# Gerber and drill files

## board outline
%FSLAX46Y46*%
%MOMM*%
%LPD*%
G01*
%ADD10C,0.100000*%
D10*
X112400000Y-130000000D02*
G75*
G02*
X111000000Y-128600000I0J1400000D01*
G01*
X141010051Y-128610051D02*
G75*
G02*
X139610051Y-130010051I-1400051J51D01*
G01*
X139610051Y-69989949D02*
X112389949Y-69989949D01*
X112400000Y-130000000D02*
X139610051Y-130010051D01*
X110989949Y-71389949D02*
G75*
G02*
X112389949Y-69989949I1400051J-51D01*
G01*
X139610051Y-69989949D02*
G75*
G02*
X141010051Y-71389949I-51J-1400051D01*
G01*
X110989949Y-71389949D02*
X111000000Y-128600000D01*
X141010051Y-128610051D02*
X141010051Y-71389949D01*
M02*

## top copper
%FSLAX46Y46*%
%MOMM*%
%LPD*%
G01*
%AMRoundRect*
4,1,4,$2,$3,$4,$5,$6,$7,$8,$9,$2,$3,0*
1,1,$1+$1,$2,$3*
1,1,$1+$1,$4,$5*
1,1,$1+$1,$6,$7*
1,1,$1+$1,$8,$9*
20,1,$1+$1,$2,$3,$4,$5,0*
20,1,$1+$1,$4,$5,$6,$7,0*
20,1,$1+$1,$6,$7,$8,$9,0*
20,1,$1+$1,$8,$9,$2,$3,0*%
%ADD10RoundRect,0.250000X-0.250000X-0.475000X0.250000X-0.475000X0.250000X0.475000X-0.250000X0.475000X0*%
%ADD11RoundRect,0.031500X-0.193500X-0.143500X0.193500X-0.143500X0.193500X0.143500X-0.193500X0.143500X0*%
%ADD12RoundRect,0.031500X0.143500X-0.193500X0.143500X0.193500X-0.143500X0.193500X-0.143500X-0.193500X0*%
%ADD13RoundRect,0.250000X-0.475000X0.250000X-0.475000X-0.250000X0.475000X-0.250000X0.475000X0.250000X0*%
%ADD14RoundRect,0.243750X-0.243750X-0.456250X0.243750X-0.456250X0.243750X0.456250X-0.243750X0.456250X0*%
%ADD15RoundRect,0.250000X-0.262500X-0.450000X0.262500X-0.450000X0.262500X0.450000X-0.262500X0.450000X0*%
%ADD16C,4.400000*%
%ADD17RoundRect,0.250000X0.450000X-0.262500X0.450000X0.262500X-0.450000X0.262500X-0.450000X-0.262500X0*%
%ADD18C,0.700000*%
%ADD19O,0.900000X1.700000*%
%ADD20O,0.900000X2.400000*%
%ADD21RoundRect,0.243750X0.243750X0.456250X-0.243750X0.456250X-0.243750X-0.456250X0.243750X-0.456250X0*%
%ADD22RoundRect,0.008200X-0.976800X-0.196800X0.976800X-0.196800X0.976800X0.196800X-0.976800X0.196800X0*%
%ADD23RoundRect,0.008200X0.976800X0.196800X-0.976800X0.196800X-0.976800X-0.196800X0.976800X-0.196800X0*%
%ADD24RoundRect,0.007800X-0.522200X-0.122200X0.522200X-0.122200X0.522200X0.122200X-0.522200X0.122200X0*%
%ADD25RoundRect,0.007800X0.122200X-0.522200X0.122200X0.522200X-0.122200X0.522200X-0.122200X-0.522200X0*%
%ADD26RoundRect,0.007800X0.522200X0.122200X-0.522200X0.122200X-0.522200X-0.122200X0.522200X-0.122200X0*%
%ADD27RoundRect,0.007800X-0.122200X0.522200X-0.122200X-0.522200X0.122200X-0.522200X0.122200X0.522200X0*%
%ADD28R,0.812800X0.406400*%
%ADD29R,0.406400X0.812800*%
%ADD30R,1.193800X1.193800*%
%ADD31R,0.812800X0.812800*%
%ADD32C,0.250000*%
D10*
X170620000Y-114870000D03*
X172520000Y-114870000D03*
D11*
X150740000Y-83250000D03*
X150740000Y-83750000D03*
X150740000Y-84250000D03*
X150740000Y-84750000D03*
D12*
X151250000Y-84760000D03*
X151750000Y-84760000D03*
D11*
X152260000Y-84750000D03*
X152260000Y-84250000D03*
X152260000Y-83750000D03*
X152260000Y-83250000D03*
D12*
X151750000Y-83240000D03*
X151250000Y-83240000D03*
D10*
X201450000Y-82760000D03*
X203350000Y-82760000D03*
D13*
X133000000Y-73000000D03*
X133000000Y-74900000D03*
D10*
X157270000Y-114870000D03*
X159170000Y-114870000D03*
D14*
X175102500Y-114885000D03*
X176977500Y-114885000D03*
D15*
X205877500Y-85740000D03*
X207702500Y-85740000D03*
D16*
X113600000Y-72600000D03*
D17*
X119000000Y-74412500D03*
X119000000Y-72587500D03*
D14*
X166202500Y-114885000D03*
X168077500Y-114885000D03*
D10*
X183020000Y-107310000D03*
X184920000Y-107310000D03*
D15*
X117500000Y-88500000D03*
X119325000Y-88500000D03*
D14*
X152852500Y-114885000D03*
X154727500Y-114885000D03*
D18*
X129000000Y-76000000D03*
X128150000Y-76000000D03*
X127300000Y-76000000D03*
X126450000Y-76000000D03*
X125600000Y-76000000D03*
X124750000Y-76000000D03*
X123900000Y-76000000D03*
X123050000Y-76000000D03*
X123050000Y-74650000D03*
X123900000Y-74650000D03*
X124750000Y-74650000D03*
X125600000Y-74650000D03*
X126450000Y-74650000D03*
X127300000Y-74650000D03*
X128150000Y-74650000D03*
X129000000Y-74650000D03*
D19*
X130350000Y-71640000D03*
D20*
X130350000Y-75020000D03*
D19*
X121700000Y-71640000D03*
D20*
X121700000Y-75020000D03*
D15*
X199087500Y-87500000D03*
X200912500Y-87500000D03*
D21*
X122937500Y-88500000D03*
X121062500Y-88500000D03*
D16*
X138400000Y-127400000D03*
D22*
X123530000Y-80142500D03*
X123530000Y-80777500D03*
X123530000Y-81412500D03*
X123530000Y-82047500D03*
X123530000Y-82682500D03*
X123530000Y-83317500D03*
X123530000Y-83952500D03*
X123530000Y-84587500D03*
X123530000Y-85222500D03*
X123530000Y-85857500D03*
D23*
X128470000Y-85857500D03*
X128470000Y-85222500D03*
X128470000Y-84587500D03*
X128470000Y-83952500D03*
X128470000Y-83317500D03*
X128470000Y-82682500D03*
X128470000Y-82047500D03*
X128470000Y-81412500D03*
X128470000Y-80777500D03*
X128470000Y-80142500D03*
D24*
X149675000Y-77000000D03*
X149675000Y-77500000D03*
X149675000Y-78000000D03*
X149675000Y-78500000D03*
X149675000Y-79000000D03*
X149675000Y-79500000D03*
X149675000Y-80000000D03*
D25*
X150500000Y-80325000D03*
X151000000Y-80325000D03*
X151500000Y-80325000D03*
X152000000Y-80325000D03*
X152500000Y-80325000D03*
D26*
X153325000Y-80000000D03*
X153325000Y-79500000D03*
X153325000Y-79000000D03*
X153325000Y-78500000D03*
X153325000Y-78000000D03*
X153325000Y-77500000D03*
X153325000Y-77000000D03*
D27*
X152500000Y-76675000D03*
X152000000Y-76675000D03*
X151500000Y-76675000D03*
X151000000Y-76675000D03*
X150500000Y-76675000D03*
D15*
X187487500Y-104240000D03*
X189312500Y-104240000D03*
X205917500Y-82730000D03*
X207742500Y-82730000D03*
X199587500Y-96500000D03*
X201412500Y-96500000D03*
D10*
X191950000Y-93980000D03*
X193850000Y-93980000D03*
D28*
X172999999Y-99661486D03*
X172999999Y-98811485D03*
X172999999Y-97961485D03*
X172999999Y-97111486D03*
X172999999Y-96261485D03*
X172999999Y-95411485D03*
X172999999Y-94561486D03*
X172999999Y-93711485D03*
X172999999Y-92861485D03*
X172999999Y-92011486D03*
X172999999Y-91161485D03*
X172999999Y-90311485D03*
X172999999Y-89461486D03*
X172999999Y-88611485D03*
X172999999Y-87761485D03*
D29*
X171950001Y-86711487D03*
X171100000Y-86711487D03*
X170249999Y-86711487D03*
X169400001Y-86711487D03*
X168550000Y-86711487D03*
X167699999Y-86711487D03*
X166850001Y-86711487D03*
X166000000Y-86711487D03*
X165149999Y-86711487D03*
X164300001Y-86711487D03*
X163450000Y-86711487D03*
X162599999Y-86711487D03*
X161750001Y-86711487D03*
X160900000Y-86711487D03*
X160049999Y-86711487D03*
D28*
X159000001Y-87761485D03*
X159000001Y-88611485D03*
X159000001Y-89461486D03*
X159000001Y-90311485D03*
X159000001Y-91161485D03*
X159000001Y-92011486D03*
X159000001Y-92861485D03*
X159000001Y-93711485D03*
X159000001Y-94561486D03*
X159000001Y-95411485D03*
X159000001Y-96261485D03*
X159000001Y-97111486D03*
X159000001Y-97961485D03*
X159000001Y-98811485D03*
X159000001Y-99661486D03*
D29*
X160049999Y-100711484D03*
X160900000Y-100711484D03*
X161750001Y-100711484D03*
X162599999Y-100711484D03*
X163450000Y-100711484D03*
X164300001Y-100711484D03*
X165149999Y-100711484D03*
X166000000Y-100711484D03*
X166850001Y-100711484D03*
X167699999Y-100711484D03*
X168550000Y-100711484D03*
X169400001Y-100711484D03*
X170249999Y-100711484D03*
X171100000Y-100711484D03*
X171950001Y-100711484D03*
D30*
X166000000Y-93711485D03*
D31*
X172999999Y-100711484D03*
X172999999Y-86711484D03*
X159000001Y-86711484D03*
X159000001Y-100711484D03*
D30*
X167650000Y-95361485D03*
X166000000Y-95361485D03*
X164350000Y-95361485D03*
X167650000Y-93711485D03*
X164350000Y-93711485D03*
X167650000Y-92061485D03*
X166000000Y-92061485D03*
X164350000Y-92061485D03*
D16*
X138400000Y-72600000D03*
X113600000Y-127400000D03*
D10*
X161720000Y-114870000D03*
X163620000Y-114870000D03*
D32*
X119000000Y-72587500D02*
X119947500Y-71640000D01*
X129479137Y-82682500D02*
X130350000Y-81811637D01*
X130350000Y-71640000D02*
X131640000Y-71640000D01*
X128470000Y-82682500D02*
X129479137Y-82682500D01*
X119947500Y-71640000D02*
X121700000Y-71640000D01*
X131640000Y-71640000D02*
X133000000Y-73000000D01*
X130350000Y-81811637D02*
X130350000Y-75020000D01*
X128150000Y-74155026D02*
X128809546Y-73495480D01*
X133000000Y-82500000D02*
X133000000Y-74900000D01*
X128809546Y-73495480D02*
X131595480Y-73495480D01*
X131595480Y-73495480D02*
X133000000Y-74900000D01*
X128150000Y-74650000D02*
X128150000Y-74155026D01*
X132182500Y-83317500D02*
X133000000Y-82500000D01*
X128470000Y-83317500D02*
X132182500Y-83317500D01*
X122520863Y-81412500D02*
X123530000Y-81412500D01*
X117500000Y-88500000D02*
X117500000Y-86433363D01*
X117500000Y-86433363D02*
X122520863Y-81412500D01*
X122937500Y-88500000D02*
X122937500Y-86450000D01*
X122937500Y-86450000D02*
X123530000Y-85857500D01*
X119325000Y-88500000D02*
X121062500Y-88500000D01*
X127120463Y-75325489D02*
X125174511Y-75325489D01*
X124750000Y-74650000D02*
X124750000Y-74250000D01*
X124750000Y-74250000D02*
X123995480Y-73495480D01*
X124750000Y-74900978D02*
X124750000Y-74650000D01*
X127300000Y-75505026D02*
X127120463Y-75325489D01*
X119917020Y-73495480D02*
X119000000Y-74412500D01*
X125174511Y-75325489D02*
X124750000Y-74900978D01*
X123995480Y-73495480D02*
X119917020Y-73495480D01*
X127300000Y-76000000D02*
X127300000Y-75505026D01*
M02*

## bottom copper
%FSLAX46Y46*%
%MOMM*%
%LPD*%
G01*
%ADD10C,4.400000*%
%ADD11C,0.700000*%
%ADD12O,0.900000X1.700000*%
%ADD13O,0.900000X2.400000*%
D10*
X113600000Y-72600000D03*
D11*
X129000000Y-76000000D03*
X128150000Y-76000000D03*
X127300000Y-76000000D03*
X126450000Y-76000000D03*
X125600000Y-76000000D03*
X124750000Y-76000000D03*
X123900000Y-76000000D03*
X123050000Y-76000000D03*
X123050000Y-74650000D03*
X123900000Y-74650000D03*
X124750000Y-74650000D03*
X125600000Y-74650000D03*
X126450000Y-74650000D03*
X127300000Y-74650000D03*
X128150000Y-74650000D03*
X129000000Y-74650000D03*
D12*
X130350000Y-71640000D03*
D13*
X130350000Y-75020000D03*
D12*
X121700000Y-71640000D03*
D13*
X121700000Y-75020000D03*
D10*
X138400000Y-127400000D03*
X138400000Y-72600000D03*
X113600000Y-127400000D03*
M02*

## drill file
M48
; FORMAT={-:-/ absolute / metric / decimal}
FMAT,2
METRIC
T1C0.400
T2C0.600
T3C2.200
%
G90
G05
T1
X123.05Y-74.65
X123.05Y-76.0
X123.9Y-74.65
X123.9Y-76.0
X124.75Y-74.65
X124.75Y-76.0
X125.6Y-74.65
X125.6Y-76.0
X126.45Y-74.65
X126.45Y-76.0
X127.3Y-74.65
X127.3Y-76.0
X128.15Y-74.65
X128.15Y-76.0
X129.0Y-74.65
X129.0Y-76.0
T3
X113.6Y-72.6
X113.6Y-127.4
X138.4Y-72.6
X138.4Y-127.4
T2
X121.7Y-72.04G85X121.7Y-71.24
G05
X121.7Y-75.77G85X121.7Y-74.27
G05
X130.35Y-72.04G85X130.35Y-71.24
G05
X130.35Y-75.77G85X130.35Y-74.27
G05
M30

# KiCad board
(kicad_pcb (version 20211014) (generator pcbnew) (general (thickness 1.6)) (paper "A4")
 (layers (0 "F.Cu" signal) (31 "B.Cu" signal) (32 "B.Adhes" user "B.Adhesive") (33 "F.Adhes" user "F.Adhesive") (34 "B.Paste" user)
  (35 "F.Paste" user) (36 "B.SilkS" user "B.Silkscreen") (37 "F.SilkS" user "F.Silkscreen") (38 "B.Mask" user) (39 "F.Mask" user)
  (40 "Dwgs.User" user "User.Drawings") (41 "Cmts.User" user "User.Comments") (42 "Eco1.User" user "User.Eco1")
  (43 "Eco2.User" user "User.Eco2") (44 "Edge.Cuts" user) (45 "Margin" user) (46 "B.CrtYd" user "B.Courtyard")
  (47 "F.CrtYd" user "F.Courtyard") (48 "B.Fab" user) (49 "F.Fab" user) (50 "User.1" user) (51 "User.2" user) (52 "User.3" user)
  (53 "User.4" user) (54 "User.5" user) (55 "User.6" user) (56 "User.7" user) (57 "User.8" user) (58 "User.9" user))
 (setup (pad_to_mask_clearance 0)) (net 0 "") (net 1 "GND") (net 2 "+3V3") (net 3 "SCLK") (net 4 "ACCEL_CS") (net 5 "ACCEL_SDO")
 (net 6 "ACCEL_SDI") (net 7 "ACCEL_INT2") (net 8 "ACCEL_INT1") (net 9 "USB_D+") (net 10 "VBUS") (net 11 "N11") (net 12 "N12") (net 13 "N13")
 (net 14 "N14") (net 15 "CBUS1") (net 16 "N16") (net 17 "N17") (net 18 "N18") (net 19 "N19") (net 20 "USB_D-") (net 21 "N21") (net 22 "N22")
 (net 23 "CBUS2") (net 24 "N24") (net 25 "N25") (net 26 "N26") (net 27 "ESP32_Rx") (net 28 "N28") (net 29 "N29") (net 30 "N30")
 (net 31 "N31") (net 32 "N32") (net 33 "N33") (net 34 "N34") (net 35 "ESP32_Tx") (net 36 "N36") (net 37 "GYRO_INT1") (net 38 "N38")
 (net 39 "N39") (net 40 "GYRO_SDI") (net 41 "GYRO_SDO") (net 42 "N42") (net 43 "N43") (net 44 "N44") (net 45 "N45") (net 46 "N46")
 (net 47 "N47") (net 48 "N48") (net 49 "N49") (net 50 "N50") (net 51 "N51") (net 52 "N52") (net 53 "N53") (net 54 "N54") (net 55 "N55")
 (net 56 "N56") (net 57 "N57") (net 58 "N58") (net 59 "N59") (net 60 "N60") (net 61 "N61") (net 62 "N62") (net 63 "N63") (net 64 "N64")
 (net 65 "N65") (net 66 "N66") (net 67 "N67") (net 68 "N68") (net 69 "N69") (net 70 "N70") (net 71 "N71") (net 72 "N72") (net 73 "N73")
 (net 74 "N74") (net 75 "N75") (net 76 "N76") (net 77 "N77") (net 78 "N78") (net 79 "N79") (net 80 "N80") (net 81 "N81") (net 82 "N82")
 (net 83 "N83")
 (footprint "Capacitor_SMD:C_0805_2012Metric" (layer "F.Cu") (at 171.57 114.87)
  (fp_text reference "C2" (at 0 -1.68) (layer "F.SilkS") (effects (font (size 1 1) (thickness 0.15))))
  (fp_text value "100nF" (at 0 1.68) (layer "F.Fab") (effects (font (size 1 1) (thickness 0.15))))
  (pad "1" smd roundrect (at -0.95 0) (size 1 1.45) (layers "F.Cu" "F.Paste" "F.Mask") (roundrect_rratio 0.25) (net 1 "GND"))
  (pad "2" smd roundrect (at 0.95 0) (size 1 1.45) (layers "F.Cu" "F.Paste" "F.Mask") (roundrect_rratio 0.25) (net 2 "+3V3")))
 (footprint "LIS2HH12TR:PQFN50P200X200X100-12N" (layer "F.Cu") (at 151.5 84)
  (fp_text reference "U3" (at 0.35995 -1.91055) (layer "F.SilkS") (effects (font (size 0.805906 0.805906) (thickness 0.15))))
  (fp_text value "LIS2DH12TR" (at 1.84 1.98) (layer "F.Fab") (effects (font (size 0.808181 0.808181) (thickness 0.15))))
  (pad "1" smd roundrect locked (at -0.76 -0.75) (size 0.45 0.35) (layers "F.Cu" "F.Paste" "F.Mask") (roundrect_rratio 0.09) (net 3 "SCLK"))
  (pad "2" smd roundrect locked (at -0.76 -0.25) (size 0.45 0.35) (layers "F.Cu" "F.Paste" "F.Mask") (roundrect_rratio 0.09)
   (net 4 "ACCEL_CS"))
  (pad "3" smd roundrect locked (at -0.76 0.25) (size 0.45 0.35) (layers "F.Cu" "F.Paste" "F.Mask") (roundrect_rratio 0.09)
   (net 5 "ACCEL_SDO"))
  (pad "4" smd roundrect locked (at -0.76 0.75) (size 0.45 0.35) (layers "F.Cu" "F.Paste" "F.Mask") (roundrect_rratio 0.09)
   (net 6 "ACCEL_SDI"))
  (pad "5" smd roundrect locked (at -0.25 0.76 90) (size 0.45 0.35) (layers "F.Cu" "F.Paste" "F.Mask") (roundrect_rratio 0.09) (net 1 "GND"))
  (pad "6" smd roundrect locked (at 0.25 0.76 90) (size 0.45 0.35) (layers "F.Cu" "F.Paste" "F.Mask") (roundrect_rratio 0.09) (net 1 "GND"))
  (pad "7" smd roundrect locked (at 0.76 0.75) (size 0.45 0.35) (layers "F.Cu" "F.Paste" "F.Mask") (roundrect_rratio 0.09) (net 1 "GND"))
  (pad "8" smd roundrect locked (at 0.76 0.25) (size 0.45 0.35) (layers "F.Cu" "F.Paste" "F.Mask") (roundrect_rratio 0.09) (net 1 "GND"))
  (pad "9" smd roundrect locked (at 0.76 -0.25) (size 0.45 0.35) (layers "F.Cu" "F.Paste" "F.Mask") (roundrect_rratio 0.09) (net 2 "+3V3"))
  (pad "10" smd roundrect locked (at 0.76 -0.75) (size 0.45 0.35) (layers "F.Cu" "F.Paste" "F.Mask") (roundrect_rratio 0.09) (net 2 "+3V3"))
  (pad "11" smd roundrect locked (at 0.25 -0.76 90) (size 0.45 0.35) (layers "F.Cu" "F.Paste" "F.Mask") (roundrect_rratio 0.09)
   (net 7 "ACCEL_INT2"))
  (pad "12" smd roundrect locked (at -0.25 -0.76 90) (size 0.45 0.35) (layers "F.Cu" "F.Paste" "F.Mask") (roundrect_rratio 0.09)
   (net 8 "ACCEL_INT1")))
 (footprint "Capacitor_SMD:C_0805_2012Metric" (layer "F.Cu") (at 202.4 82.76)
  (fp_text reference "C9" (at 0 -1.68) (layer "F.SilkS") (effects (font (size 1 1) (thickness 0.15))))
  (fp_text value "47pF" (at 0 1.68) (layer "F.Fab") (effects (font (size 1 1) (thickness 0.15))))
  (pad "1" smd roundrect (at -0.95 0) (size 1 1.45) (layers "F.Cu" "F.Paste" "F.Mask") (roundrect_rratio 0.25) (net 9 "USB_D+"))
  (pad "2" smd roundrect (at 0.95 0) (size 1 1.45) (layers "F.Cu" "F.Paste" "F.Mask") (roundrect_rratio 0.25) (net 1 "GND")))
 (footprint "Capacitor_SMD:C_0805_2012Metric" (layer "F.Cu") (at 133 73.95 -90)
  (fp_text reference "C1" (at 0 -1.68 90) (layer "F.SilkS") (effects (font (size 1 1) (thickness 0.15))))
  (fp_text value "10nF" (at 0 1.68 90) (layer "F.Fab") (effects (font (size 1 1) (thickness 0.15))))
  (pad "1" smd roundrect (at -0.95 0 270) (size 1 1.45) (layers "F.Cu" "F.Paste" "F.Mask") (roundrect_rratio 0.25) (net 1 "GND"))
  (pad "2" smd roundrect (at 0.95 0 270) (size 1 1.45) (layers "F.Cu" "F.Paste" "F.Mask") (roundrect_rratio 0.25) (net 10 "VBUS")))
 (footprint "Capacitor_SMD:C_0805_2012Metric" (layer "F.Cu") (at 158.22 114.87)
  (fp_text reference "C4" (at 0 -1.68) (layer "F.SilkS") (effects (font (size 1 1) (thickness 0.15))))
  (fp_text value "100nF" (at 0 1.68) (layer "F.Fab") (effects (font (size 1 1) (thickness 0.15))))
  (pad "1" smd roundrect (at -0.95 0) (size 1 1.45) (layers "F.Cu" "F.Paste" "F.Mask") (roundrect_rratio 0.25) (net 1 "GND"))
  (pad "2" smd roundrect (at 0.95 0) (size 1 1.45) (layers "F.Cu" "F.Paste" "F.Mask") (roundrect_rratio 0.25) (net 2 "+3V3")))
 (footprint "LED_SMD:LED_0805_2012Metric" (layer "F.Cu") (at 176.04 114.885)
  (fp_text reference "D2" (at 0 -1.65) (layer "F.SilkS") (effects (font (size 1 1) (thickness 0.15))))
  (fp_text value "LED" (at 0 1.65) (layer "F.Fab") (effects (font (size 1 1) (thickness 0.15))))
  (pad "1" smd roundrect (at -0.9375 0) (size 0.975 1.4) (layers "F.Cu" "F.Paste" "F.Mask") (roundrect_rratio 0.25) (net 1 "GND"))
  (pad "2" smd roundrect (at 0.9375 0) (size 0.975 1.4) (layers "F.Cu" "F.Paste" "F.Mask") (roundrect_rratio 0.25) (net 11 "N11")))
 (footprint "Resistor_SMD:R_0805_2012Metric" (layer "F.Cu") (at 206.79 85.74)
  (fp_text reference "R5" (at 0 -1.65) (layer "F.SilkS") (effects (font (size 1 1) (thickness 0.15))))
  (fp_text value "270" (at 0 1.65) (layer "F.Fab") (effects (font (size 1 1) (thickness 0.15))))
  (pad "1" smd roundrect (at -0.9125 0) (size 1.025 1.4) (layers "F.Cu" "F.Paste" "F.Mask") (roundrect_rratio 0.243902) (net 2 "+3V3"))
  (pad "2" smd roundrect (at 0.9125 0) (size 1.025 1.4) (layers "F.Cu" "F.Paste" "F.Mask") (roundrect_rratio 0.243902) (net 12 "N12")))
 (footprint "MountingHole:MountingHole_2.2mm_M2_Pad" (layer "F.Cu") (at 113.6 72.6)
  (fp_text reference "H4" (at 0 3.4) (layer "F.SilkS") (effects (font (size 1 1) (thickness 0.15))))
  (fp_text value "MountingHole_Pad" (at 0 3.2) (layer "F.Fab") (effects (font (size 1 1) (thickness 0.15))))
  (pad "1" thru_hole circle (at 0 0) (size 4.4 4.4) (drill 2.2) (layers *.Cu *.Mask) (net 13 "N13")))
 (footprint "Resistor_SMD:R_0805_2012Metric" (layer "F.Cu") (at 119 73.5 90)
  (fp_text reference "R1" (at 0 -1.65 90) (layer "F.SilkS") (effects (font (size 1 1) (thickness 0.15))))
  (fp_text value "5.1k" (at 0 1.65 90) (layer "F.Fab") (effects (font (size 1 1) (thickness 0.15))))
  (pad "1" smd roundrect (at -0.9125 0 90) (size 1.025 1.4) (layers "F.Cu" "F.Paste" "F.Mask") (roundrect_rratio 0.243902) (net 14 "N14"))
  (pad "2" smd roundrect (at 0.9125 0 90) (size 1.025 1.4) (layers "F.Cu" "F.Paste" "F.Mask") (roundrect_rratio 0.243902) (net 1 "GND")))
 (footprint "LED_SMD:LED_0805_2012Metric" (layer "F.Cu") (at 167.14 114.885)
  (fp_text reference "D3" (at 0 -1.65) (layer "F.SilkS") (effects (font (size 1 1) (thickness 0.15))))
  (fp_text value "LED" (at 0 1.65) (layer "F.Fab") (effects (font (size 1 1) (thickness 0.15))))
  (pad "1" smd roundrect (at -0.9375 0) (size 0.975 1.4) (layers "F.Cu" "F.Paste" "F.Mask") (roundrect_rratio 0.25) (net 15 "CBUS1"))
  (pad "2" smd roundrect (at 0.9375 0) (size 0.975 1.4) (layers "F.Cu" "F.Paste" "F.Mask") (roundrect_rratio 0.25) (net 12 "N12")))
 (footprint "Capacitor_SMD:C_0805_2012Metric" (layer "F.Cu") (at 183.97 107.31)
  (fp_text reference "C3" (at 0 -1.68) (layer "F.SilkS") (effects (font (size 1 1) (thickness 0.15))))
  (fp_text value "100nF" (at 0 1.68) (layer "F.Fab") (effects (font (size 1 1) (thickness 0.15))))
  (pad "1" smd roundrect (at -0.95 0) (size 1 1.45) (layers "F.Cu" "F.Paste" "F.Mask") (roundrect_rratio 0.25) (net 2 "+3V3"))
  (pad "2" smd roundrect (at 0.95 0) (size 1 1.45) (layers "F.Cu" "F.Paste" "F.Mask") (roundrect_rratio 0.25) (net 1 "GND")))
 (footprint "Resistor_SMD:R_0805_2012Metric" (layer "F.Cu") (at 118.4125 88.5)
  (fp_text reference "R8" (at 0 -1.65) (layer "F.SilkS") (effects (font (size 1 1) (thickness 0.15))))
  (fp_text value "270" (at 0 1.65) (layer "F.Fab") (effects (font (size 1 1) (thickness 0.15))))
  (pad "1" smd roundrect (at -0.9125 0) (size 1.025 1.4) (layers "F.Cu" "F.Paste" "F.Mask") (roundrect_rratio 0.243902) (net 2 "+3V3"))
  (pad "2" smd roundrect (at 0.9125 0) (size 1.025 1.4) (layers "F.Cu" "F.Paste" "F.Mask") (roundrect_rratio 0.243902) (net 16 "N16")))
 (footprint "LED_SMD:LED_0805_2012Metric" (layer "F.Cu") (at 153.79 114.885)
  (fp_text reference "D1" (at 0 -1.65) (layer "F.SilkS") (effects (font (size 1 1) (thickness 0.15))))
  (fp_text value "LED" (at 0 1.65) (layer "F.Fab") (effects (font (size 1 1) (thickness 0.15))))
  (pad "1" smd roundrect (at -0.9375 0) (size 0.975 1.4) (layers "F.Cu" "F.Paste" "F.Mask") (roundrect_rratio 0.25) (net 1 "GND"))
  (pad "2" smd roundrect (at 0.9375 0) (size 0.975 1.4) (layers "F.Cu" "F.Paste" "F.Mask") (roundrect_rratio 0.25) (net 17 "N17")))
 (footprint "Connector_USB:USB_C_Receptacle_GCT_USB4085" (layer "F.Cu") (at 129 76 180)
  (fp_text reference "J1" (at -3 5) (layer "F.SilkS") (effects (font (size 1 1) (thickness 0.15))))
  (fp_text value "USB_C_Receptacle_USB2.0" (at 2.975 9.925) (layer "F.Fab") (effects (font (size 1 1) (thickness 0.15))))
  (pad "A1" thru_hole circle (at 0 0 180) (size 0.7 0.7) (drill 0.4) (layers *.Cu *.Mask) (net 1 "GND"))
  (pad "A4" thru_hole circle (at 0.85 0 180) (size 0.7 0.7) (drill 0.4) (layers *.Cu *.Mask) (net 10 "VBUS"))
  (pad "A5" thru_hole circle (at 1.7 0 180) (size 0.7 0.7) (drill 0.4) (layers *.Cu *.Mask) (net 14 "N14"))
  (pad "A6" thru_hole circle (at 2.55 0 180) (size 0.7 0.7) (drill 0.4) (layers *.Cu *.Mask) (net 9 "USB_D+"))
  (pad "A7" thru_hole circle (at 3.4 0 180) (size 0.7 0.7) (drill 0.4) (layers *.Cu *.Mask) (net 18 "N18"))
  (pad "A8" thru_hole circle (at 4.25 0 180) (size 0.7 0.7) (drill 0.4) (layers *.Cu *.Mask) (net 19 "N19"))
  (pad "A9" thru_hole circle (at 5.1 0 180) (size 0.7 0.7) (drill 0.4) (layers *.Cu *.Mask) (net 10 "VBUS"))
  (pad "A12" thru_hole circle (at 5.95 0 180) (size 0.7 0.7) (drill 0.4) (layers *.Cu *.Mask) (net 1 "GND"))
  (pad "B1" thru_hole circle (at 5.95 1.35 180) (size 0.7 0.7) (drill 0.4) (layers *.Cu *.Mask) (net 1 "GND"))
  (pad "B4" thru_hole circle (at 5.1 1.35 180) (size 0.7 0.7) (drill 0.4) (layers *.Cu *.Mask) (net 10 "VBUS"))
  (pad "B5" thru_hole circle (at 4.25 1.35 180) (size 0.7 0.7) (drill 0.4) (layers *.Cu *.Mask) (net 14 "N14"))
  (pad "B6" thru_hole circle (at 3.4 1.35 180) (size 0.7 0.7) (drill 0.4) (layers *.Cu *.Mask) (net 9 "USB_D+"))
  (pad "B7" thru_hole circle (at 2.55 1.35 180) (size 0.7 0.7) (drill 0.4) (layers *.Cu *.Mask) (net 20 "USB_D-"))
  (pad "B8" thru_hole circle (at 1.7 1.35 180) (size 0.7 0.7) (drill 0.4) (layers *.Cu *.Mask) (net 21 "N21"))
  (pad "B9" thru_hole circle (at 0.85 1.35 180) (size 0.7 0.7) (drill 0.4) (layers *.Cu *.Mask) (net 10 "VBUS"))
  (pad "B12" thru_hole circle (at 0 1.35 180) (size 0.7 0.7) (drill 0.4) (layers *.Cu *.Mask) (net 1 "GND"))
  (pad "S1" thru_hole oval (at -1.35 4.36 180) (size 0.9 1.7) (drill oval 0.6 1.4) (layers *.Cu *.Mask) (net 1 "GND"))
  (pad "S1" thru_hole oval (at -1.35 0.98 180) (size 0.9 2.4) (drill oval 0.6 2.1) (layers *.Cu *.Mask) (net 1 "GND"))
  (pad "S1" thru_hole oval (at 7.3 4.36 180) (size 0.9 1.7) (drill oval 0.6 1.4) (layers *.Cu *.Mask) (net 1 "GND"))
  (pad "S1" thru_hole oval (at 7.3 0.98 180) (size 0.9 2.4) (drill oval 0.6 2.1) (layers *.Cu *.Mask) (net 1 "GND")))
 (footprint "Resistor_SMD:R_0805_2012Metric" (layer "F.Cu") (at 200 87.5)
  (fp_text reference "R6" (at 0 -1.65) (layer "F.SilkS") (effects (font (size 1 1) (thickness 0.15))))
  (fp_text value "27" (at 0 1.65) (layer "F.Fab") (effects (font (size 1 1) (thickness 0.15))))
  (pad "1" smd roundrect (at -0.9125 0) (size 1.025 1.4) (layers "F.Cu" "F.Paste" "F.Mask") (roundrect_rratio 0.243902) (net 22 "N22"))
  (pad "2" smd roundrect (at 0.9125 0) (size 1.025 1.4) (layers "F.Cu" "F.Paste" "F.Mask") (roundrect_rratio 0.243902) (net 9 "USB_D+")))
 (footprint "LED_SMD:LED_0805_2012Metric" (layer "F.Cu") (at 122 88.5 180)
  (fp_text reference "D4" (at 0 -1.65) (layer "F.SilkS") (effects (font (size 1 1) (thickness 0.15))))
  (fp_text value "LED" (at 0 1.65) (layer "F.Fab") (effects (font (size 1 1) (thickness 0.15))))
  (pad "1" smd roundrect (at -0.9375 0 180) (size 0.975 1.4) (layers "F.Cu" "F.Paste" "F.Mask") (roundrect_rratio 0.25) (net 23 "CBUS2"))
  (pad "2" smd roundrect (at 0.9375 0 180) (size 0.975 1.4) (layers "F.Cu" "F.Paste" "F.Mask") (roundrect_rratio 0.25) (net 16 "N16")))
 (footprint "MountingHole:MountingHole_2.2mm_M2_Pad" (layer "F.Cu") (at 138.4 127.4)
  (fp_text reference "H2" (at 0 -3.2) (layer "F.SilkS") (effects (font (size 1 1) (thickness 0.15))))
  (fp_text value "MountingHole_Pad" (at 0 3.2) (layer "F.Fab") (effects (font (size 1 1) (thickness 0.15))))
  (pad "1" thru_hole circle (at 0 0) (size 4.4 4.4) (drill 2.2) (layers *.Cu *.Mask) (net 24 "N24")))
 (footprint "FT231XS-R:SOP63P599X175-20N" (layer "F.Cu") (at 126 83)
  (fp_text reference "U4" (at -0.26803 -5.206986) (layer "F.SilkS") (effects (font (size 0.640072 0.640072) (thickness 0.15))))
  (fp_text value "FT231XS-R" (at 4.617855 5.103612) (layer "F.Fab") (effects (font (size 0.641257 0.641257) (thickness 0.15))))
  (pad "1" smd roundrect locked (at -2.47 -2.8575) (size 1.97 0.41) (layers "F.Cu" "F.Paste" "F.Mask") (roundrect_rratio 0.02)
   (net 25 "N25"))
  (pad "2" smd roundrect locked (at -2.47 -2.2225) (size 1.97 0.41) (layers "F.Cu" "F.Paste" "F.Mask") (roundrect_rratio 0.02)
   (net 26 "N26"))
  (pad "3" smd roundrect locked (at -2.47 -1.5875) (size 1.97 0.41) (layers "F.Cu" "F.Paste" "F.Mask") (roundrect_rratio 0.02)
   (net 2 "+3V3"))
  (pad "4" smd roundrect locked (at -2.47 -0.9525) (size 1.97 0.41) (layers "F.Cu" "F.Paste" "F.Mask") (roundrect_rratio 0.02)
   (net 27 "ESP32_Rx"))
  (pad "5" smd roundrect locked (at -2.47 -0.3175) (size 1.97 0.41) (layers "F.Cu" "F.Paste" "F.Mask") (roundrect_rratio 0.02)
   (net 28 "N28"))
  (pad "6" smd roundrect locked (at -2.47 0.3175) (size 1.97 0.41) (layers "F.Cu" "F.Paste" "F.Mask") (roundrect_rratio 0.02) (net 1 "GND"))
  (pad "7" smd roundrect locked (at -2.47 0.9525) (size 1.97 0.41) (layers "F.Cu" "F.Paste" "F.Mask") (roundrect_rratio 0.02) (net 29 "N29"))
  (pad "8" smd roundrect locked (at -2.47 1.5875) (size 1.97 0.41) (layers "F.Cu" "F.Paste" "F.Mask") (roundrect_rratio 0.02) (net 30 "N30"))
  (pad "9" smd roundrect locked (at -2.47 2.2225) (size 1.97 0.41) (layers "F.Cu" "F.Paste" "F.Mask") (roundrect_rratio 0.02) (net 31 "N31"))
  (pad "10" smd roundrect locked (at -2.47 2.8575) (size 1.97 0.41) (layers "F.Cu" "F.Paste" "F.Mask") (roundrect_rratio 0.02)
   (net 23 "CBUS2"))
  (pad "11" smd roundrect locked (at 2.47 2.8575 180) (size 1.97 0.41) (layers "F.Cu" "F.Paste" "F.Mask") (roundrect_rratio 0.02)
   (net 22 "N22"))
  (pad "12" smd roundrect locked (at 2.47 2.2225 180) (size 1.97 0.41) (layers "F.Cu" "F.Paste" "F.Mask") (roundrect_rratio 0.02)
   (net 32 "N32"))
  (pad "13" smd roundrect locked (at 2.47 1.5875 180) (size 1.97 0.41) (layers "F.Cu" "F.Paste" "F.Mask") (roundrect_rratio 0.02)
   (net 2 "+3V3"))
  (pad "14" smd roundrect locked (at 2.47 0.9525 180) (size 1.97 0.41) (layers "F.Cu" "F.Paste" "F.Mask") (roundrect_rratio 0.02)
   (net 2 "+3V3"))
  (pad "15" smd roundrect locked (at 2.47 0.3175 180) (size 1.97 0.41) (layers "F.Cu" "F.Paste" "F.Mask") (roundrect_rratio 0.02)
   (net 10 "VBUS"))
  (pad "16" smd roundrect locked (at 2.47 -0.3175 180) (size 1.97 0.41) (layers "F.Cu" "F.Paste" "F.Mask") (roundrect_rratio 0.02)
   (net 1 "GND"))
  (pad "17" smd roundrect locked (at 2.47 -0.9525 180) (size 1.97 0.41) (layers "F.Cu" "F.Paste" "F.Mask") (roundrect_rratio 0.02)
   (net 15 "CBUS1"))
  (pad "18" smd roundrect locked (at 2.47 -1.5875 180) (size 1.97 0.41) (layers "F.Cu" "F.Paste" "F.Mask") (roundrect_rratio 0.02)
   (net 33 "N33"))
  (pad "19" smd roundrect locked (at 2.47 -2.2225 180) (size 1.97 0.41) (layers "F.Cu" "F.Paste" "F.Mask") (roundrect_rratio 0.02)
   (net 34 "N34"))
  (pad "20" smd roundrect locked (at 2.47 -2.8575 180) (size 1.97 0.41) (layers "F.Cu" "F.Paste" "F.Mask") (roundrect_rratio 0.02)
   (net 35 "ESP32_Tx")))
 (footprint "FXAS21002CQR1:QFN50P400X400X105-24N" (layer "F.Cu") (at 151.5 78.5)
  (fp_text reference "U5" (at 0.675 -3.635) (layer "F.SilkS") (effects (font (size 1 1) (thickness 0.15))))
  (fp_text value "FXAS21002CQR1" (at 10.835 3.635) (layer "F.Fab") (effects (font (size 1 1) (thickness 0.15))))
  (pad "1" smd roundrect locked (at -1.825 -1.5) (size 1.06 0.26) (layers "F.Cu" "F.Paste" "F.Mask") (roundrect_rratio 0.03) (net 1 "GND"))
  (pad "2" smd roundrect locked (at -1.825 -1) (size 1.06 0.26) (layers "F.Cu" "F.Paste" "F.Mask") (roundrect_rratio 0.03) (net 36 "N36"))
  (pad "3" smd roundrect locked (at -1.825 -0.5) (size 1.06 0.26) (layers "F.Cu" "F.Paste" "F.Mask") (roundrect_rratio 0.03)
   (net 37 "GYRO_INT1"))
  (pad "4" smd roundrect locked (at -1.825 0) (size 1.06 0.26) (layers "F.Cu" "F.Paste" "F.Mask") (roundrect_rratio 0.03) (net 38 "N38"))
  (pad "5" smd roundrect locked (at -1.825 0.5) (size 1.06 0.26) (layers "F.Cu" "F.Paste" "F.Mask") (roundrect_rratio 0.03) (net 1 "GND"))
  (pad "6" smd roundrect locked (at -1.825 1) (size 1.06 0.26) (layers "F.Cu" "F.Paste" "F.Mask") (roundrect_rratio 0.03) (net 1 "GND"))
  (pad "7" smd roundrect locked (at -1.825 1.5) (size 1.06 0.26) (layers "F.Cu" "F.Paste" "F.Mask") (roundrect_rratio 0.03) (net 1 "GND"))
  (pad "8" smd roundrect locked (at -1 1.825 90) (size 1.06 0.26) (layers "F.Cu" "F.Paste" "F.Mask") (roundrect_rratio 0.03) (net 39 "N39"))
  (pad "9" smd roundrect locked (at -0.5 1.825 90) (size 1.06 0.26) (layers "F.Cu" "F.Paste" "F.Mask") (roundrect_rratio 0.03) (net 1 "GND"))
  (pad "10" smd roundrect locked (at 0 1.825 90) (size 1.06 0.26) (layers "F.Cu" "F.Paste" "F.Mask") (roundrect_rratio 0.03) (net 1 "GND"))
  (pad "11" smd roundrect locked (at 0.5 1.825 90) (size 1.06 0.26) (layers "F.Cu" "F.Paste" "F.Mask") (roundrect_rratio 0.03)
   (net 3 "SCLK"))
  (pad "12" smd roundrect locked (at 1 1.825 90) (size 1.06 0.26) (layers "F.Cu" "F.Paste" "F.Mask") (roundrect_rratio 0.03)
   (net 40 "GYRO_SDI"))
  (pad "13" smd roundrect locked (at 1.825 1.5 180) (size 1.06 0.26) (layers "F.Cu" "F.Paste" "F.Mask") (roundrect_rratio 0.03)
   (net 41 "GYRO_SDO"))
  (pad "14" smd roundrect locked (at 1.825 1 180) (size 1.06 0.26) (layers "F.Cu" "F.Paste" "F.Mask") (roundrect_rratio 0.03) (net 1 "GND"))
  (pad "15" smd roundrect locked (at 1.825 0.5 180) (size 1.06 0.26) (layers "F.Cu" "F.Paste" "F.Mask") (roundrect_rratio 0.03)
   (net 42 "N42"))
  (pad "16" smd roundrect locked (at 1.825 0 180) (size 1.06 0.26) (layers "F.Cu" "F.Paste" "F.Mask") (roundrect_rratio 0.03) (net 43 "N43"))
  (pad "17" smd roundrect locked (at 1.825 -0.5 180) (size 1.06 0.26) (layers "F.Cu" "F.Paste" "F.Mask") (roundrect_rratio 0.03)
   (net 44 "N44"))
  (pad "18" smd roundrect locked (at 1.825 -1 180) (size 1.06 0.26) (layers "F.Cu" "F.Paste" "F.Mask") (roundrect_rratio 0.03)
   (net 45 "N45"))
  (pad "19" smd roundrect locked (at 1.825 -1.5 180) (size 1.06 0.26) (layers "F.Cu" "F.Paste" "F.Mask") (roundrect_rratio 0.03)
   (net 1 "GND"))
  (pad "20" smd roundrect locked (at 1 -1.825 270) (size 1.06 0.26) (layers "F.Cu" "F.Paste" "F.Mask") (roundrect_rratio 0.03) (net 1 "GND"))
  (pad "21" smd roundrect locked (at 0.5 -1.825 270) (size 1.06 0.26) (layers "F.Cu" "F.Paste" "F.Mask") (roundrect_rratio 0.03)
   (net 1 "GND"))
  (pad "22" smd roundrect locked (at 0 -1.825 270) (size 1.06 0.26) (layers "F.Cu" "F.Paste" "F.Mask") (roundrect_rratio 0.03) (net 1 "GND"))
  (pad "23" smd roundrect locked (at -0.5 -1.825 270) (size 1.06 0.26) (layers "F.Cu" "F.Paste" "F.Mask") (roundrect_rratio 0.03)
   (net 1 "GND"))
  (pad "24" smd roundrect locked (at -1 -1.825 270) (size 1.06 0.26) (layers "F.Cu" "F.Paste" "F.Mask") (roundrect_rratio 0.03)
   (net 1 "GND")))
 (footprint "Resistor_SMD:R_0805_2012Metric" (layer "F.Cu") (at 188.4 104.24)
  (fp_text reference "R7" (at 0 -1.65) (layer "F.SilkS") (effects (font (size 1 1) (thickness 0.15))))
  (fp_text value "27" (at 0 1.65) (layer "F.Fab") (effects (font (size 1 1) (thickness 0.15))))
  (pad "1" smd roundrect (at -0.9125 0) (size 1.025 1.4) (layers "F.Cu" "F.Paste" "F.Mask") (roundrect_rratio 0.243902) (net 32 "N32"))
  (pad "2" smd roundrect (at 0.9125 0) (size 1.025 1.4) (layers "F.Cu" "F.Paste" "F.Mask") (roundrect_rratio 0.243902) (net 20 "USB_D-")))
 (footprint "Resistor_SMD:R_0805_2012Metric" (layer "F.Cu") (at 206.83 82.73)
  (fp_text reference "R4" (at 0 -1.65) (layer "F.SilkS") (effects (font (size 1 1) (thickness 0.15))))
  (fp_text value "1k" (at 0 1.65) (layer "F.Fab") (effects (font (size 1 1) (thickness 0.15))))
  (pad "1" smd roundrect (at -0.9125 0) (size 1.025 1.4) (layers "F.Cu" "F.Paste" "F.Mask") (roundrect_rratio 0.243902) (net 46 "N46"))
  (pad "2" smd roundrect (at 0.9125 0) (size 1.025 1.4) (layers "F.Cu" "F.Paste" "F.Mask") (roundrect_rratio 0.243902) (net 11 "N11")))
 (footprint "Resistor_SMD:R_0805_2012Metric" (layer "F.Cu") (at 200.5 96.5)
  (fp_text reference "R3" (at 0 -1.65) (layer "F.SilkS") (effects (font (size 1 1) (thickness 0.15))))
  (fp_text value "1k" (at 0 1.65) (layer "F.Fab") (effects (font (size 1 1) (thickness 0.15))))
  (pad "1" smd roundrect (at -0.9125 0) (size 1.025 1.4) (layers "F.Cu" "F.Paste" "F.Mask") (roundrect_rratio 0.243902) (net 17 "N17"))
  (pad "2" smd roundrect (at 0.9125 0) (size 1.025 1.4) (layers "F.Cu" "F.Paste" "F.Mask") (roundrect_rratio 0.243902) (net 2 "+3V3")))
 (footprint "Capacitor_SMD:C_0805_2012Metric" (layer "F.Cu") (at 192.9 93.98)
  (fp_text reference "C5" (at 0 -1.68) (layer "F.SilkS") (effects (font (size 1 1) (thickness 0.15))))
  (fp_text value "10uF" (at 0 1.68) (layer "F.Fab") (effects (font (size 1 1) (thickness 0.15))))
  (pad "1" smd roundrect (at -0.95 0) (size 1 1.45) (layers "F.Cu" "F.Paste" "F.Mask") (roundrect_rratio 0.25) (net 1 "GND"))
  (pad "2" smd roundrect (at 0.95 0) (size 1 1.45) (layers "F.Cu" "F.Paste" "F.Mask") (roundrect_rratio 0.25) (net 2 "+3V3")))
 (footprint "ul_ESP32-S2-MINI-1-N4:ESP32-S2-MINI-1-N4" (layer "F.Cu") (at 166 96 180)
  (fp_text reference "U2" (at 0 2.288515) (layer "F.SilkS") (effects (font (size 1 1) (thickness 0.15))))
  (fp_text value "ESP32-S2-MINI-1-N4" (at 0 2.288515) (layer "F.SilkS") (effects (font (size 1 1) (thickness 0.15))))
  (pad "1" smd rect locked (at -6.999999 -3.661486 180) (size 0.8128 0.4064) (layers "F.Cu" "F.Paste" "F.Mask") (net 1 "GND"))
  (pad "2" smd rect locked (at -6.999999 -2.811485 180) (size 0.8128 0.4064) (layers "F.Cu" "F.Paste" "F.Mask") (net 1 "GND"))
  (pad "3" smd rect locked (at -6.999999 -1.961485 180) (size 0.8128 0.4064) (layers "F.Cu" "F.Paste" "F.Mask") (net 2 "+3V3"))
  (pad "4" smd rect locked (at -6.999999 -1.111486 180) (size 0.8128 0.4064) (layers "F.Cu" "F.Paste" "F.Mask") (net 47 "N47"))
  (pad "5" smd rect locked (at -6.999999 -0.261485 180) (size 0.8128 0.4064) (layers "F.Cu" "F.Paste" "F.Mask") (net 46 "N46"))
  (pad "6" smd rect locked (at -6.999999 0.588515 180) (size 0.8128 0.4064) (layers "F.Cu" "F.Paste" "F.Mask") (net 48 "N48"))
  (pad "7" smd rect locked (at -6.999999 1.438514 180) (size 0.8128 0.4064) (layers "F.Cu" "F.Paste" "F.Mask") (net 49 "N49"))
  (pad "8" smd rect locked (at -6.999999 2.288515 180) (size 0.8128 0.4064) (layers "F.Cu" "F.Paste" "F.Mask") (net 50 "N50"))
  (pad "9" smd rect locked (at -6.999999 3.138515 180) (size 0.8128 0.4064) (layers "F.Cu" "F.Paste" "F.Mask") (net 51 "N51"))
  (pad "10" smd rect locked (at -6.999999 3.988514 180) (size 0.8128 0.4064) (layers "F.Cu" "F.Paste" "F.Mask") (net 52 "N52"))
  (pad "11" smd rect locked (at -6.999999 4.838515 180) (size 0.8128 0.4064) (layers "F.Cu" "F.Paste" "F.Mask") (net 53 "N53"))
  (pad "12" smd rect locked (at -6.999999 5.688515 180) (size 0.8128 0.4064) (layers "F.Cu" "F.Paste" "F.Mask") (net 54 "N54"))
  (pad "13" smd rect locked (at -6.999999 6.538514 180) (size 0.8128 0.4064) (layers "F.Cu" "F.Paste" "F.Mask") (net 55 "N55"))
  (pad "14" smd rect locked (at -6.999999 7.388515 180) (size 0.8128 0.4064) (layers "F.Cu" "F.Paste" "F.Mask") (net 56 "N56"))
  (pad "15" smd rect locked (at -6.999999 8.238515 180) (size 0.8128 0.4064) (layers "F.Cu" "F.Paste" "F.Mask") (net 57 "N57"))
  (pad "16" smd rect locked (at -5.950001 9.288513 180) (size 0.4064 0.8128) (layers "F.Cu" "F.Paste" "F.Mask") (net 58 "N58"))
  (pad "17" smd rect locked (at -5.1 9.288513 180) (size 0.4064 0.8128) (layers "F.Cu" "F.Paste" "F.Mask") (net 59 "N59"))
  (pad "18" smd rect locked (at -4.249999 9.288513 180) (size 0.4064 0.8128) (layers "F.Cu" "F.Paste" "F.Mask") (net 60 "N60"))
  (pad "19" smd rect locked (at -3.400001 9.288513 180) (size 0.4064 0.8128) (layers "F.Cu" "F.Paste" "F.Mask") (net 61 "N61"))
  (pad "20" smd rect locked (at -2.55 9.288513 180) (size 0.4064 0.8128) (layers "F.Cu" "F.Paste" "F.Mask") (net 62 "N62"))
  (pad "21" smd rect locked (at -1.699999 9.288513 180) (size 0.4064 0.8128) (layers "F.Cu" "F.Paste" "F.Mask") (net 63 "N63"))
  (pad "22" smd rect locked (at -0.850001 9.288513 180) (size 0.4064 0.8128) (layers "F.Cu" "F.Paste" "F.Mask") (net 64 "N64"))
  (pad "23" smd rect locked (at 0 9.288513 180) (size 0.4064 0.8128) (layers "F.Cu" "F.Paste" "F.Mask") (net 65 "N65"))
  (pad "24" smd rect locked (at 0.850001 9.288513 180) (size 0.4064 0.8128) (layers "F.Cu" "F.Paste" "F.Mask") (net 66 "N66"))
  (pad "25" smd rect locked (at 1.699999 9.288513 180) (size 0.4064 0.8128) (layers "F.Cu" "F.Paste" "F.Mask") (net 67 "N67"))
  (pad "26" smd rect locked (at 2.55 9.288513 180) (size 0.4064 0.8128) (layers "F.Cu" "F.Paste" "F.Mask") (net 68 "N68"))
  (pad "27" smd rect locked (at 3.400001 9.288513 180) (size 0.4064 0.8128) (layers "F.Cu" "F.Paste" "F.Mask") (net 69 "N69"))
  (pad "28" smd rect locked (at 4.249999 9.288513 180) (size 0.4064 0.8128) (layers "F.Cu" "F.Paste" "F.Mask") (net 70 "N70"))
  (pad "29" smd rect locked (at 5.1 9.288513 180) (size 0.4064 0.8128) (layers "F.Cu" "F.Paste" "F.Mask") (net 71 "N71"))
  (pad "30" smd rect locked (at 5.950001 9.288513 180) (size 0.4064 0.8128) (layers "F.Cu" "F.Paste" "F.Mask") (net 1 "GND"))
  (pad "31" smd rect locked (at 6.999999 8.238515 180) (size 0.8128 0.4064) (layers "F.Cu" "F.Paste" "F.Mask") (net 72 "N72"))
  (pad "32" smd rect locked (at 6.999999 7.388515 180) (size 0.8128 0.4064) (layers "F.Cu" "F.Paste" "F.Mask") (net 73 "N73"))
  (pad "33" smd rect locked (at 6.999999 6.538514 180) (size 0.8128 0.4064) (layers "F.Cu" "F.Paste" "F.Mask") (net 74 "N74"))
  (pad "34" smd rect locked (at 6.999999 5.688515 180) (size 0.8128 0.4064) (layers "F.Cu" "F.Paste" "F.Mask") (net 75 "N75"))
  (pad "35" smd rect locked (at 6.999999 4.838515 180) (size 0.8128 0.4064) (layers "F.Cu" "F.Paste" "F.Mask") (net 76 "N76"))
  (pad "36" smd rect locked (at 6.999999 3.988514 180) (size 0.8128 0.4064) (layers "F.Cu" "F.Paste" "F.Mask") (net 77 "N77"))
  (pad "37" smd rect locked (at 6.999999 3.138515 180) (size 0.8128 0.4064) (layers "F.Cu" "F.Paste" "F.Mask") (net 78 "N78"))
  (pad "38" smd rect locked (at 6.999999 2.288515 180) (size 0.8128 0.4064) (layers "F.Cu" "F.Paste" "F.Mask") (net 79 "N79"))
  (pad "39" smd rect locked (at 6.999999 1.438514 180) (size 0.8128 0.4064) (layers "F.Cu" "F.Paste" "F.Mask") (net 35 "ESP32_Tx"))
  (pad "40" smd rect locked (at 6.999999 0.588515 180) (size 0.8128 0.4064) (layers "F.Cu" "F.Paste" "F.Mask") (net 27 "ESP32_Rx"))
  (pad "41" smd rect locked (at 6.999999 -0.261485 180) (size 0.8128 0.4064) (layers "F.Cu" "F.Paste" "F.Mask") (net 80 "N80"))
  (pad "42" smd rect locked (at 6.999999 -1.111486 180) (size 0.8128 0.4064) (layers "F.Cu" "F.Paste" "F.Mask") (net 1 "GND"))
  (pad "43" smd rect locked (at 6.999999 -1.961485 180) (size 0.8128 0.4064) (layers "F.Cu" "F.Paste" "F.Mask") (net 1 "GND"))
  (pad "44" smd rect locked (at 6.999999 -2.811485 180) (size 0.8128 0.4064) (layers "F.Cu" "F.Paste" "F.Mask") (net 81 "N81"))
  (pad "45" smd rect locked (at 6.999999 -3.661486 180) (size 0.8128 0.4064) (layers "F.Cu" "F.Paste" "F.Mask") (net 2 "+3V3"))
  (pad "46" smd rect locked (at 5.950001 -4.711484 180) (size 0.4064 0.8128) (layers "F.Cu" "F.Paste" "F.Mask") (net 1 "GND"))
  (pad "47" smd rect locked (at 5.1 -4.711484 180) (size 0.4064 0.8128) (layers "F.Cu" "F.Paste" "F.Mask") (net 1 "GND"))
  (pad "48" smd rect locked (at 4.249999 -4.711484 180) (size 0.4064 0.8128) (layers "F.Cu" "F.Paste" "F.Mask") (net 1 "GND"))
  (pad "49" smd rect locked (at 3.400001 -4.711484 180) (size 0.4064 0.8128) (layers "F.Cu" "F.Paste" "F.Mask") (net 1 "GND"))
  (pad "50" smd rect locked (at 2.55 -4.711484 180) (size 0.4064 0.8128) (layers "F.Cu" "F.Paste" "F.Mask") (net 1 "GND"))
  (pad "51" smd rect locked (at 1.699999 -4.711484 180) (size 0.4064 0.8128) (layers "F.Cu" "F.Paste" "F.Mask") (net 1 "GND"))
  (pad "52" smd rect locked (at 0.850001 -4.711484 180) (size 0.4064 0.8128) (layers "F.Cu" "F.Paste" "F.Mask") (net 1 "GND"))
  (pad "53" smd rect locked (at 0 -4.711484 180) (size 0.4064 0.8128) (layers "F.Cu" "F.Paste" "F.Mask") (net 1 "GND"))
  (pad "54" smd rect locked (at -0.850001 -4.711484 180) (size 0.4064 0.8128) (layers "F.Cu" "F.Paste" "F.Mask") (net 1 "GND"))
  (pad "55" smd rect locked (at -1.699999 -4.711484 180) (size 0.4064 0.8128) (layers "F.Cu" "F.Paste" "F.Mask") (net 1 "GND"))
  (pad "56" smd rect locked (at -2.55 -4.711484 180) (size 0.4064 0.8128) (layers "F.Cu" "F.Paste" "F.Mask") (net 1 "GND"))
  (pad "57" smd rect locked (at -3.400001 -4.711484 180) (size 0.4064 0.8128) (layers "F.Cu" "F.Paste" "F.Mask") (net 1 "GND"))
  (pad "58" smd rect locked (at -4.249999 -4.711484 180) (size 0.4064 0.8128) (layers "F.Cu" "F.Paste" "F.Mask") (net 1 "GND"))
  (pad "59" smd rect locked (at -5.1 -4.711484 180) (size 0.4064 0.8128) (layers "F.Cu" "F.Paste" "F.Mask") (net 1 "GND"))
  (pad "60" smd rect locked (at -5.950001 -4.711484 180) (size 0.4064 0.8128) (layers "F.Cu" "F.Paste" "F.Mask") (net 1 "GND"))
  (pad "61" smd rect locked (at 0 2.288515 180) (size 1.1938 1.1938) (layers "F.Cu" "F.Paste" "F.Mask") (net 1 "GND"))
  (pad "62" smd rect locked (at -6.999999 -4.711484 180) (size 0.8128 0.8128) (layers "F.Cu" "F.Paste" "F.Mask") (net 1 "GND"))
  (pad "63" smd rect locked (at -6.999999 9.288516 180) (size 0.8128 0.8128) (layers "F.Cu" "F.Paste" "F.Mask") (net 1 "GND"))
  (pad "64" smd rect locked (at 6.999999 9.288516 180) (size 0.8128 0.8128) (layers "F.Cu" "F.Paste" "F.Mask") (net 1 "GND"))
  (pad "65" smd rect locked (at 6.999999 -4.711484 180) (size 0.8128 0.8128) (layers "F.Cu" "F.Paste" "F.Mask") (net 1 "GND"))
  (pad "66" smd rect locked (at -1.65 0.638515 180) (size 1.1938 1.1938) (layers "F.Cu" "F.Paste" "F.Mask") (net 1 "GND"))
  (pad "67" smd rect locked (at 0 0.638515 180) (size 1.1938 1.1938) (layers "F.Cu" "F.Paste" "F.Mask") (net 1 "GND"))
  (pad "68" smd rect locked (at 1.65 0.638515 180) (size 1.1938 1.1938) (layers "F.Cu" "F.Paste" "F.Mask") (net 1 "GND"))
  (pad "69" smd rect locked (at -1.65 2.288515 180) (size 1.1938 1.1938) (layers "F.Cu" "F.Paste" "F.Mask") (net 1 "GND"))
  (pad "70" smd rect locked (at 1.65 2.288515 180) (size 1.1938 1.1938) (layers "F.Cu" "F.Paste" "F.Mask") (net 1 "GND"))
  (pad "71" smd rect locked (at -1.65 3.938515 180) (size 1.1938 1.1938) (layers "F.Cu" "F.Paste" "F.Mask") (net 1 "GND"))
  (pad "72" smd rect locked (at 0 3.938515 180) (size 1.1938 1.1938) (layers "F.Cu" "F.Paste" "F.Mask") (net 1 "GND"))
  (pad "73" smd rect locked (at 1.65 3.938515 180) (size 1.1938 1.1938) (layers "F.Cu" "F.Paste" "F.Mask") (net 1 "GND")))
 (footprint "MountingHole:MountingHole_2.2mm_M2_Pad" (layer "F.Cu") (at 138.4 72.6)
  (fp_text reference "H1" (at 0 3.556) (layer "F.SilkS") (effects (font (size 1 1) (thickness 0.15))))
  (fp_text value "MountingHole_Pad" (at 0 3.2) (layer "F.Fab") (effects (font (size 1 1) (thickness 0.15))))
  (pad "1" thru_hole circle (at 0 0) (size 4.4 4.4) (drill 2.2) (layers *.Cu *.Mask) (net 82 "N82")))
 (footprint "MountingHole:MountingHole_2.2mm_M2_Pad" (layer "F.Cu") (at 113.6 127.4)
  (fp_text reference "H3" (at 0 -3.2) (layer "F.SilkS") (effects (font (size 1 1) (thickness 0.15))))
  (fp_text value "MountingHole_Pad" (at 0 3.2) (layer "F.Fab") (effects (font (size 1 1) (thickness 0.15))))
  (pad "1" thru_hole circle (at 0 0) (size 4.4 4.4) (drill 2.2) (layers *.Cu *.Mask) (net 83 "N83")))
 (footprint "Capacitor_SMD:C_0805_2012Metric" (layer "F.Cu") (at 162.67 114.87)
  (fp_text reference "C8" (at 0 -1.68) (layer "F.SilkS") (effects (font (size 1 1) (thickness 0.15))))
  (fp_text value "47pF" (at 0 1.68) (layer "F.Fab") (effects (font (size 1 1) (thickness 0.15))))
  (pad "1" smd roundrect (at -0.95 0) (size 1 1.45) (layers "F.Cu" "F.Paste" "F.Mask") (roundrect_rratio 0.25) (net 20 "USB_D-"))
  (pad "2" smd roundrect (at 0.95 0) (size 1 1.45) (layers "F.Cu" "F.Paste" "F.Mask") (roundrect_rratio 0.25) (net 1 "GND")))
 (gr_arc (start 112.4 130) (mid 111.410051 129.589949) (end 111 128.6) (layer "Edge.Cuts") (width 0.1))
 (gr_arc (start 141.010051 128.610051) (mid 140.6 129.6) (end 139.610051 130.010051) (layer "Edge.Cuts") (width 0.1))
 (gr_line (start 139.610051 69.989949) (end 112.389949 69.989949) (layer "Edge.Cuts") (width 0.1))
 (gr_line (start 112.4 130) (end 139.610051 130.010051) (layer "Edge.Cuts") (width 0.1))
 (gr_arc (start 110.989949 71.389949) (mid 111.4 70.4) (end 112.389949 69.989949) (layer "Edge.Cuts") (width 0.1))
 (gr_arc (start 139.610051 69.989949) (mid 140.6 70.4) (end 141.010051 71.389949) (layer "Edge.Cuts") (width 0.1))
 (gr_line (start 110.989949 71.389949) (end 111 128.6) (layer "Edge.Cuts") (width 0.1))
 (gr_line (start 141.010051 128.610051) (end 141.010051 71.389949) (layer "Edge.Cuts") (width 0.1))
 (segment (start 119 72.5875) (end 119.9475 71.64) (width 0.25) (layer "F.Cu") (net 1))
 (segment (start 129.479137 82.6825) (end 130.35 81.811637) (width 0.25) (layer "F.Cu") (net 1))
 (segment (start 130.35 71.64) (end 131.64 71.64) (width 0.25) (layer "F.Cu") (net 1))
 (segment (start 128.47 82.6825) (end 129.479137 82.6825) (width 0.25) (layer "F.Cu") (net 1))
 (segment (start 119.9475 71.64) (end 121.7 71.64) (width 0.25) (layer "F.Cu") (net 1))
 (segment (start 131.64 71.64) (end 133 73) (width 0.25) (layer "F.Cu") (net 1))
 (segment (start 130.35 81.811637) (end 130.35 75.02) (width 0.25) (layer "F.Cu") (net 1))
 (segment (start 128.15 74.155026) (end 128.809546 73.49548) (width 0.25) (layer "F.Cu") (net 10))
 (segment (start 133 82.5) (end 133 74.9) (width 0.25) (layer "F.Cu") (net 10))
 (segment (start 128.809546 73.49548) (end 131.59548 73.49548) (width 0.25) (layer "F.Cu") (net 10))
 (segment (start 131.59548 73.49548) (end 133 74.9) (width 0.25) (layer "F.Cu") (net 10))
 (segment (start 128.15 74.65) (end 128.15 74.155026) (width 0.25) (layer "F.Cu") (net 10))
 (segment (start 132.1825 83.3175) (end 133 82.5) (width 0.25) (layer "F.Cu") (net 10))
 (segment (start 128.47 83.3175) (end 132.1825 83.3175) (width 0.25) (layer "F.Cu") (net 10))
 (segment (start 122.520863 81.4125) (end 123.53 81.4125) (width 0.25) (layer "F.Cu") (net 2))
 (segment (start 117.5 88.5) (end 117.5 86.433363) (width 0.25) (layer "F.Cu") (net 2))
 (segment (start 117.5 86.433363) (end 122.520863 81.4125) (width 0.25) (layer "F.Cu") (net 2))
 (segment (start 122.9375 88.5) (end 122.9375 86.45) (width 0.25) (layer "F.Cu") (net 23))
 (segment (start 122.9375 86.45) (end 123.53 85.8575) (width 0.25) (layer "F.Cu") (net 23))
 (segment (start 119.325 88.5) (end 121.0625 88.5) (width 0.25) (layer "F.Cu") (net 16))
 (segment (start 127.120463 75.325489) (end 125.174511 75.325489) (width 0.25) (layer "F.Cu") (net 14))
 (segment (start 124.75 74.65) (end 124.75 74.25) (width 0.25) (layer "F.Cu") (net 14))
 (segment (start 124.75 74.25) (end 123.99548 73.49548) (width 0.25) (layer "F.Cu") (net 14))
 (segment (start 124.75 74.900978) (end 124.75 74.65) (width 0.25) (layer "F.Cu") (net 14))
 (segment (start 127.3 75.505026) (end 127.120463 75.325489) (width 0.25) (layer "F.Cu") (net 14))
 (segment (start 119.91702 73.49548) (end 119 74.4125) (width 0.25) (layer "F.Cu") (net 14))
 (segment (start 125.174511 75.325489) (end 124.75 74.900978) (width 0.25) (layer "F.Cu") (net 14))
 (segment (start 123.99548 73.49548) (end 119.91702 73.49548) (width 0.25) (layer "F.Cu") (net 14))
 (segment (start 127.3 76) (end 127.3 75.505026) (width 0.25) (layer "F.Cu") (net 14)))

